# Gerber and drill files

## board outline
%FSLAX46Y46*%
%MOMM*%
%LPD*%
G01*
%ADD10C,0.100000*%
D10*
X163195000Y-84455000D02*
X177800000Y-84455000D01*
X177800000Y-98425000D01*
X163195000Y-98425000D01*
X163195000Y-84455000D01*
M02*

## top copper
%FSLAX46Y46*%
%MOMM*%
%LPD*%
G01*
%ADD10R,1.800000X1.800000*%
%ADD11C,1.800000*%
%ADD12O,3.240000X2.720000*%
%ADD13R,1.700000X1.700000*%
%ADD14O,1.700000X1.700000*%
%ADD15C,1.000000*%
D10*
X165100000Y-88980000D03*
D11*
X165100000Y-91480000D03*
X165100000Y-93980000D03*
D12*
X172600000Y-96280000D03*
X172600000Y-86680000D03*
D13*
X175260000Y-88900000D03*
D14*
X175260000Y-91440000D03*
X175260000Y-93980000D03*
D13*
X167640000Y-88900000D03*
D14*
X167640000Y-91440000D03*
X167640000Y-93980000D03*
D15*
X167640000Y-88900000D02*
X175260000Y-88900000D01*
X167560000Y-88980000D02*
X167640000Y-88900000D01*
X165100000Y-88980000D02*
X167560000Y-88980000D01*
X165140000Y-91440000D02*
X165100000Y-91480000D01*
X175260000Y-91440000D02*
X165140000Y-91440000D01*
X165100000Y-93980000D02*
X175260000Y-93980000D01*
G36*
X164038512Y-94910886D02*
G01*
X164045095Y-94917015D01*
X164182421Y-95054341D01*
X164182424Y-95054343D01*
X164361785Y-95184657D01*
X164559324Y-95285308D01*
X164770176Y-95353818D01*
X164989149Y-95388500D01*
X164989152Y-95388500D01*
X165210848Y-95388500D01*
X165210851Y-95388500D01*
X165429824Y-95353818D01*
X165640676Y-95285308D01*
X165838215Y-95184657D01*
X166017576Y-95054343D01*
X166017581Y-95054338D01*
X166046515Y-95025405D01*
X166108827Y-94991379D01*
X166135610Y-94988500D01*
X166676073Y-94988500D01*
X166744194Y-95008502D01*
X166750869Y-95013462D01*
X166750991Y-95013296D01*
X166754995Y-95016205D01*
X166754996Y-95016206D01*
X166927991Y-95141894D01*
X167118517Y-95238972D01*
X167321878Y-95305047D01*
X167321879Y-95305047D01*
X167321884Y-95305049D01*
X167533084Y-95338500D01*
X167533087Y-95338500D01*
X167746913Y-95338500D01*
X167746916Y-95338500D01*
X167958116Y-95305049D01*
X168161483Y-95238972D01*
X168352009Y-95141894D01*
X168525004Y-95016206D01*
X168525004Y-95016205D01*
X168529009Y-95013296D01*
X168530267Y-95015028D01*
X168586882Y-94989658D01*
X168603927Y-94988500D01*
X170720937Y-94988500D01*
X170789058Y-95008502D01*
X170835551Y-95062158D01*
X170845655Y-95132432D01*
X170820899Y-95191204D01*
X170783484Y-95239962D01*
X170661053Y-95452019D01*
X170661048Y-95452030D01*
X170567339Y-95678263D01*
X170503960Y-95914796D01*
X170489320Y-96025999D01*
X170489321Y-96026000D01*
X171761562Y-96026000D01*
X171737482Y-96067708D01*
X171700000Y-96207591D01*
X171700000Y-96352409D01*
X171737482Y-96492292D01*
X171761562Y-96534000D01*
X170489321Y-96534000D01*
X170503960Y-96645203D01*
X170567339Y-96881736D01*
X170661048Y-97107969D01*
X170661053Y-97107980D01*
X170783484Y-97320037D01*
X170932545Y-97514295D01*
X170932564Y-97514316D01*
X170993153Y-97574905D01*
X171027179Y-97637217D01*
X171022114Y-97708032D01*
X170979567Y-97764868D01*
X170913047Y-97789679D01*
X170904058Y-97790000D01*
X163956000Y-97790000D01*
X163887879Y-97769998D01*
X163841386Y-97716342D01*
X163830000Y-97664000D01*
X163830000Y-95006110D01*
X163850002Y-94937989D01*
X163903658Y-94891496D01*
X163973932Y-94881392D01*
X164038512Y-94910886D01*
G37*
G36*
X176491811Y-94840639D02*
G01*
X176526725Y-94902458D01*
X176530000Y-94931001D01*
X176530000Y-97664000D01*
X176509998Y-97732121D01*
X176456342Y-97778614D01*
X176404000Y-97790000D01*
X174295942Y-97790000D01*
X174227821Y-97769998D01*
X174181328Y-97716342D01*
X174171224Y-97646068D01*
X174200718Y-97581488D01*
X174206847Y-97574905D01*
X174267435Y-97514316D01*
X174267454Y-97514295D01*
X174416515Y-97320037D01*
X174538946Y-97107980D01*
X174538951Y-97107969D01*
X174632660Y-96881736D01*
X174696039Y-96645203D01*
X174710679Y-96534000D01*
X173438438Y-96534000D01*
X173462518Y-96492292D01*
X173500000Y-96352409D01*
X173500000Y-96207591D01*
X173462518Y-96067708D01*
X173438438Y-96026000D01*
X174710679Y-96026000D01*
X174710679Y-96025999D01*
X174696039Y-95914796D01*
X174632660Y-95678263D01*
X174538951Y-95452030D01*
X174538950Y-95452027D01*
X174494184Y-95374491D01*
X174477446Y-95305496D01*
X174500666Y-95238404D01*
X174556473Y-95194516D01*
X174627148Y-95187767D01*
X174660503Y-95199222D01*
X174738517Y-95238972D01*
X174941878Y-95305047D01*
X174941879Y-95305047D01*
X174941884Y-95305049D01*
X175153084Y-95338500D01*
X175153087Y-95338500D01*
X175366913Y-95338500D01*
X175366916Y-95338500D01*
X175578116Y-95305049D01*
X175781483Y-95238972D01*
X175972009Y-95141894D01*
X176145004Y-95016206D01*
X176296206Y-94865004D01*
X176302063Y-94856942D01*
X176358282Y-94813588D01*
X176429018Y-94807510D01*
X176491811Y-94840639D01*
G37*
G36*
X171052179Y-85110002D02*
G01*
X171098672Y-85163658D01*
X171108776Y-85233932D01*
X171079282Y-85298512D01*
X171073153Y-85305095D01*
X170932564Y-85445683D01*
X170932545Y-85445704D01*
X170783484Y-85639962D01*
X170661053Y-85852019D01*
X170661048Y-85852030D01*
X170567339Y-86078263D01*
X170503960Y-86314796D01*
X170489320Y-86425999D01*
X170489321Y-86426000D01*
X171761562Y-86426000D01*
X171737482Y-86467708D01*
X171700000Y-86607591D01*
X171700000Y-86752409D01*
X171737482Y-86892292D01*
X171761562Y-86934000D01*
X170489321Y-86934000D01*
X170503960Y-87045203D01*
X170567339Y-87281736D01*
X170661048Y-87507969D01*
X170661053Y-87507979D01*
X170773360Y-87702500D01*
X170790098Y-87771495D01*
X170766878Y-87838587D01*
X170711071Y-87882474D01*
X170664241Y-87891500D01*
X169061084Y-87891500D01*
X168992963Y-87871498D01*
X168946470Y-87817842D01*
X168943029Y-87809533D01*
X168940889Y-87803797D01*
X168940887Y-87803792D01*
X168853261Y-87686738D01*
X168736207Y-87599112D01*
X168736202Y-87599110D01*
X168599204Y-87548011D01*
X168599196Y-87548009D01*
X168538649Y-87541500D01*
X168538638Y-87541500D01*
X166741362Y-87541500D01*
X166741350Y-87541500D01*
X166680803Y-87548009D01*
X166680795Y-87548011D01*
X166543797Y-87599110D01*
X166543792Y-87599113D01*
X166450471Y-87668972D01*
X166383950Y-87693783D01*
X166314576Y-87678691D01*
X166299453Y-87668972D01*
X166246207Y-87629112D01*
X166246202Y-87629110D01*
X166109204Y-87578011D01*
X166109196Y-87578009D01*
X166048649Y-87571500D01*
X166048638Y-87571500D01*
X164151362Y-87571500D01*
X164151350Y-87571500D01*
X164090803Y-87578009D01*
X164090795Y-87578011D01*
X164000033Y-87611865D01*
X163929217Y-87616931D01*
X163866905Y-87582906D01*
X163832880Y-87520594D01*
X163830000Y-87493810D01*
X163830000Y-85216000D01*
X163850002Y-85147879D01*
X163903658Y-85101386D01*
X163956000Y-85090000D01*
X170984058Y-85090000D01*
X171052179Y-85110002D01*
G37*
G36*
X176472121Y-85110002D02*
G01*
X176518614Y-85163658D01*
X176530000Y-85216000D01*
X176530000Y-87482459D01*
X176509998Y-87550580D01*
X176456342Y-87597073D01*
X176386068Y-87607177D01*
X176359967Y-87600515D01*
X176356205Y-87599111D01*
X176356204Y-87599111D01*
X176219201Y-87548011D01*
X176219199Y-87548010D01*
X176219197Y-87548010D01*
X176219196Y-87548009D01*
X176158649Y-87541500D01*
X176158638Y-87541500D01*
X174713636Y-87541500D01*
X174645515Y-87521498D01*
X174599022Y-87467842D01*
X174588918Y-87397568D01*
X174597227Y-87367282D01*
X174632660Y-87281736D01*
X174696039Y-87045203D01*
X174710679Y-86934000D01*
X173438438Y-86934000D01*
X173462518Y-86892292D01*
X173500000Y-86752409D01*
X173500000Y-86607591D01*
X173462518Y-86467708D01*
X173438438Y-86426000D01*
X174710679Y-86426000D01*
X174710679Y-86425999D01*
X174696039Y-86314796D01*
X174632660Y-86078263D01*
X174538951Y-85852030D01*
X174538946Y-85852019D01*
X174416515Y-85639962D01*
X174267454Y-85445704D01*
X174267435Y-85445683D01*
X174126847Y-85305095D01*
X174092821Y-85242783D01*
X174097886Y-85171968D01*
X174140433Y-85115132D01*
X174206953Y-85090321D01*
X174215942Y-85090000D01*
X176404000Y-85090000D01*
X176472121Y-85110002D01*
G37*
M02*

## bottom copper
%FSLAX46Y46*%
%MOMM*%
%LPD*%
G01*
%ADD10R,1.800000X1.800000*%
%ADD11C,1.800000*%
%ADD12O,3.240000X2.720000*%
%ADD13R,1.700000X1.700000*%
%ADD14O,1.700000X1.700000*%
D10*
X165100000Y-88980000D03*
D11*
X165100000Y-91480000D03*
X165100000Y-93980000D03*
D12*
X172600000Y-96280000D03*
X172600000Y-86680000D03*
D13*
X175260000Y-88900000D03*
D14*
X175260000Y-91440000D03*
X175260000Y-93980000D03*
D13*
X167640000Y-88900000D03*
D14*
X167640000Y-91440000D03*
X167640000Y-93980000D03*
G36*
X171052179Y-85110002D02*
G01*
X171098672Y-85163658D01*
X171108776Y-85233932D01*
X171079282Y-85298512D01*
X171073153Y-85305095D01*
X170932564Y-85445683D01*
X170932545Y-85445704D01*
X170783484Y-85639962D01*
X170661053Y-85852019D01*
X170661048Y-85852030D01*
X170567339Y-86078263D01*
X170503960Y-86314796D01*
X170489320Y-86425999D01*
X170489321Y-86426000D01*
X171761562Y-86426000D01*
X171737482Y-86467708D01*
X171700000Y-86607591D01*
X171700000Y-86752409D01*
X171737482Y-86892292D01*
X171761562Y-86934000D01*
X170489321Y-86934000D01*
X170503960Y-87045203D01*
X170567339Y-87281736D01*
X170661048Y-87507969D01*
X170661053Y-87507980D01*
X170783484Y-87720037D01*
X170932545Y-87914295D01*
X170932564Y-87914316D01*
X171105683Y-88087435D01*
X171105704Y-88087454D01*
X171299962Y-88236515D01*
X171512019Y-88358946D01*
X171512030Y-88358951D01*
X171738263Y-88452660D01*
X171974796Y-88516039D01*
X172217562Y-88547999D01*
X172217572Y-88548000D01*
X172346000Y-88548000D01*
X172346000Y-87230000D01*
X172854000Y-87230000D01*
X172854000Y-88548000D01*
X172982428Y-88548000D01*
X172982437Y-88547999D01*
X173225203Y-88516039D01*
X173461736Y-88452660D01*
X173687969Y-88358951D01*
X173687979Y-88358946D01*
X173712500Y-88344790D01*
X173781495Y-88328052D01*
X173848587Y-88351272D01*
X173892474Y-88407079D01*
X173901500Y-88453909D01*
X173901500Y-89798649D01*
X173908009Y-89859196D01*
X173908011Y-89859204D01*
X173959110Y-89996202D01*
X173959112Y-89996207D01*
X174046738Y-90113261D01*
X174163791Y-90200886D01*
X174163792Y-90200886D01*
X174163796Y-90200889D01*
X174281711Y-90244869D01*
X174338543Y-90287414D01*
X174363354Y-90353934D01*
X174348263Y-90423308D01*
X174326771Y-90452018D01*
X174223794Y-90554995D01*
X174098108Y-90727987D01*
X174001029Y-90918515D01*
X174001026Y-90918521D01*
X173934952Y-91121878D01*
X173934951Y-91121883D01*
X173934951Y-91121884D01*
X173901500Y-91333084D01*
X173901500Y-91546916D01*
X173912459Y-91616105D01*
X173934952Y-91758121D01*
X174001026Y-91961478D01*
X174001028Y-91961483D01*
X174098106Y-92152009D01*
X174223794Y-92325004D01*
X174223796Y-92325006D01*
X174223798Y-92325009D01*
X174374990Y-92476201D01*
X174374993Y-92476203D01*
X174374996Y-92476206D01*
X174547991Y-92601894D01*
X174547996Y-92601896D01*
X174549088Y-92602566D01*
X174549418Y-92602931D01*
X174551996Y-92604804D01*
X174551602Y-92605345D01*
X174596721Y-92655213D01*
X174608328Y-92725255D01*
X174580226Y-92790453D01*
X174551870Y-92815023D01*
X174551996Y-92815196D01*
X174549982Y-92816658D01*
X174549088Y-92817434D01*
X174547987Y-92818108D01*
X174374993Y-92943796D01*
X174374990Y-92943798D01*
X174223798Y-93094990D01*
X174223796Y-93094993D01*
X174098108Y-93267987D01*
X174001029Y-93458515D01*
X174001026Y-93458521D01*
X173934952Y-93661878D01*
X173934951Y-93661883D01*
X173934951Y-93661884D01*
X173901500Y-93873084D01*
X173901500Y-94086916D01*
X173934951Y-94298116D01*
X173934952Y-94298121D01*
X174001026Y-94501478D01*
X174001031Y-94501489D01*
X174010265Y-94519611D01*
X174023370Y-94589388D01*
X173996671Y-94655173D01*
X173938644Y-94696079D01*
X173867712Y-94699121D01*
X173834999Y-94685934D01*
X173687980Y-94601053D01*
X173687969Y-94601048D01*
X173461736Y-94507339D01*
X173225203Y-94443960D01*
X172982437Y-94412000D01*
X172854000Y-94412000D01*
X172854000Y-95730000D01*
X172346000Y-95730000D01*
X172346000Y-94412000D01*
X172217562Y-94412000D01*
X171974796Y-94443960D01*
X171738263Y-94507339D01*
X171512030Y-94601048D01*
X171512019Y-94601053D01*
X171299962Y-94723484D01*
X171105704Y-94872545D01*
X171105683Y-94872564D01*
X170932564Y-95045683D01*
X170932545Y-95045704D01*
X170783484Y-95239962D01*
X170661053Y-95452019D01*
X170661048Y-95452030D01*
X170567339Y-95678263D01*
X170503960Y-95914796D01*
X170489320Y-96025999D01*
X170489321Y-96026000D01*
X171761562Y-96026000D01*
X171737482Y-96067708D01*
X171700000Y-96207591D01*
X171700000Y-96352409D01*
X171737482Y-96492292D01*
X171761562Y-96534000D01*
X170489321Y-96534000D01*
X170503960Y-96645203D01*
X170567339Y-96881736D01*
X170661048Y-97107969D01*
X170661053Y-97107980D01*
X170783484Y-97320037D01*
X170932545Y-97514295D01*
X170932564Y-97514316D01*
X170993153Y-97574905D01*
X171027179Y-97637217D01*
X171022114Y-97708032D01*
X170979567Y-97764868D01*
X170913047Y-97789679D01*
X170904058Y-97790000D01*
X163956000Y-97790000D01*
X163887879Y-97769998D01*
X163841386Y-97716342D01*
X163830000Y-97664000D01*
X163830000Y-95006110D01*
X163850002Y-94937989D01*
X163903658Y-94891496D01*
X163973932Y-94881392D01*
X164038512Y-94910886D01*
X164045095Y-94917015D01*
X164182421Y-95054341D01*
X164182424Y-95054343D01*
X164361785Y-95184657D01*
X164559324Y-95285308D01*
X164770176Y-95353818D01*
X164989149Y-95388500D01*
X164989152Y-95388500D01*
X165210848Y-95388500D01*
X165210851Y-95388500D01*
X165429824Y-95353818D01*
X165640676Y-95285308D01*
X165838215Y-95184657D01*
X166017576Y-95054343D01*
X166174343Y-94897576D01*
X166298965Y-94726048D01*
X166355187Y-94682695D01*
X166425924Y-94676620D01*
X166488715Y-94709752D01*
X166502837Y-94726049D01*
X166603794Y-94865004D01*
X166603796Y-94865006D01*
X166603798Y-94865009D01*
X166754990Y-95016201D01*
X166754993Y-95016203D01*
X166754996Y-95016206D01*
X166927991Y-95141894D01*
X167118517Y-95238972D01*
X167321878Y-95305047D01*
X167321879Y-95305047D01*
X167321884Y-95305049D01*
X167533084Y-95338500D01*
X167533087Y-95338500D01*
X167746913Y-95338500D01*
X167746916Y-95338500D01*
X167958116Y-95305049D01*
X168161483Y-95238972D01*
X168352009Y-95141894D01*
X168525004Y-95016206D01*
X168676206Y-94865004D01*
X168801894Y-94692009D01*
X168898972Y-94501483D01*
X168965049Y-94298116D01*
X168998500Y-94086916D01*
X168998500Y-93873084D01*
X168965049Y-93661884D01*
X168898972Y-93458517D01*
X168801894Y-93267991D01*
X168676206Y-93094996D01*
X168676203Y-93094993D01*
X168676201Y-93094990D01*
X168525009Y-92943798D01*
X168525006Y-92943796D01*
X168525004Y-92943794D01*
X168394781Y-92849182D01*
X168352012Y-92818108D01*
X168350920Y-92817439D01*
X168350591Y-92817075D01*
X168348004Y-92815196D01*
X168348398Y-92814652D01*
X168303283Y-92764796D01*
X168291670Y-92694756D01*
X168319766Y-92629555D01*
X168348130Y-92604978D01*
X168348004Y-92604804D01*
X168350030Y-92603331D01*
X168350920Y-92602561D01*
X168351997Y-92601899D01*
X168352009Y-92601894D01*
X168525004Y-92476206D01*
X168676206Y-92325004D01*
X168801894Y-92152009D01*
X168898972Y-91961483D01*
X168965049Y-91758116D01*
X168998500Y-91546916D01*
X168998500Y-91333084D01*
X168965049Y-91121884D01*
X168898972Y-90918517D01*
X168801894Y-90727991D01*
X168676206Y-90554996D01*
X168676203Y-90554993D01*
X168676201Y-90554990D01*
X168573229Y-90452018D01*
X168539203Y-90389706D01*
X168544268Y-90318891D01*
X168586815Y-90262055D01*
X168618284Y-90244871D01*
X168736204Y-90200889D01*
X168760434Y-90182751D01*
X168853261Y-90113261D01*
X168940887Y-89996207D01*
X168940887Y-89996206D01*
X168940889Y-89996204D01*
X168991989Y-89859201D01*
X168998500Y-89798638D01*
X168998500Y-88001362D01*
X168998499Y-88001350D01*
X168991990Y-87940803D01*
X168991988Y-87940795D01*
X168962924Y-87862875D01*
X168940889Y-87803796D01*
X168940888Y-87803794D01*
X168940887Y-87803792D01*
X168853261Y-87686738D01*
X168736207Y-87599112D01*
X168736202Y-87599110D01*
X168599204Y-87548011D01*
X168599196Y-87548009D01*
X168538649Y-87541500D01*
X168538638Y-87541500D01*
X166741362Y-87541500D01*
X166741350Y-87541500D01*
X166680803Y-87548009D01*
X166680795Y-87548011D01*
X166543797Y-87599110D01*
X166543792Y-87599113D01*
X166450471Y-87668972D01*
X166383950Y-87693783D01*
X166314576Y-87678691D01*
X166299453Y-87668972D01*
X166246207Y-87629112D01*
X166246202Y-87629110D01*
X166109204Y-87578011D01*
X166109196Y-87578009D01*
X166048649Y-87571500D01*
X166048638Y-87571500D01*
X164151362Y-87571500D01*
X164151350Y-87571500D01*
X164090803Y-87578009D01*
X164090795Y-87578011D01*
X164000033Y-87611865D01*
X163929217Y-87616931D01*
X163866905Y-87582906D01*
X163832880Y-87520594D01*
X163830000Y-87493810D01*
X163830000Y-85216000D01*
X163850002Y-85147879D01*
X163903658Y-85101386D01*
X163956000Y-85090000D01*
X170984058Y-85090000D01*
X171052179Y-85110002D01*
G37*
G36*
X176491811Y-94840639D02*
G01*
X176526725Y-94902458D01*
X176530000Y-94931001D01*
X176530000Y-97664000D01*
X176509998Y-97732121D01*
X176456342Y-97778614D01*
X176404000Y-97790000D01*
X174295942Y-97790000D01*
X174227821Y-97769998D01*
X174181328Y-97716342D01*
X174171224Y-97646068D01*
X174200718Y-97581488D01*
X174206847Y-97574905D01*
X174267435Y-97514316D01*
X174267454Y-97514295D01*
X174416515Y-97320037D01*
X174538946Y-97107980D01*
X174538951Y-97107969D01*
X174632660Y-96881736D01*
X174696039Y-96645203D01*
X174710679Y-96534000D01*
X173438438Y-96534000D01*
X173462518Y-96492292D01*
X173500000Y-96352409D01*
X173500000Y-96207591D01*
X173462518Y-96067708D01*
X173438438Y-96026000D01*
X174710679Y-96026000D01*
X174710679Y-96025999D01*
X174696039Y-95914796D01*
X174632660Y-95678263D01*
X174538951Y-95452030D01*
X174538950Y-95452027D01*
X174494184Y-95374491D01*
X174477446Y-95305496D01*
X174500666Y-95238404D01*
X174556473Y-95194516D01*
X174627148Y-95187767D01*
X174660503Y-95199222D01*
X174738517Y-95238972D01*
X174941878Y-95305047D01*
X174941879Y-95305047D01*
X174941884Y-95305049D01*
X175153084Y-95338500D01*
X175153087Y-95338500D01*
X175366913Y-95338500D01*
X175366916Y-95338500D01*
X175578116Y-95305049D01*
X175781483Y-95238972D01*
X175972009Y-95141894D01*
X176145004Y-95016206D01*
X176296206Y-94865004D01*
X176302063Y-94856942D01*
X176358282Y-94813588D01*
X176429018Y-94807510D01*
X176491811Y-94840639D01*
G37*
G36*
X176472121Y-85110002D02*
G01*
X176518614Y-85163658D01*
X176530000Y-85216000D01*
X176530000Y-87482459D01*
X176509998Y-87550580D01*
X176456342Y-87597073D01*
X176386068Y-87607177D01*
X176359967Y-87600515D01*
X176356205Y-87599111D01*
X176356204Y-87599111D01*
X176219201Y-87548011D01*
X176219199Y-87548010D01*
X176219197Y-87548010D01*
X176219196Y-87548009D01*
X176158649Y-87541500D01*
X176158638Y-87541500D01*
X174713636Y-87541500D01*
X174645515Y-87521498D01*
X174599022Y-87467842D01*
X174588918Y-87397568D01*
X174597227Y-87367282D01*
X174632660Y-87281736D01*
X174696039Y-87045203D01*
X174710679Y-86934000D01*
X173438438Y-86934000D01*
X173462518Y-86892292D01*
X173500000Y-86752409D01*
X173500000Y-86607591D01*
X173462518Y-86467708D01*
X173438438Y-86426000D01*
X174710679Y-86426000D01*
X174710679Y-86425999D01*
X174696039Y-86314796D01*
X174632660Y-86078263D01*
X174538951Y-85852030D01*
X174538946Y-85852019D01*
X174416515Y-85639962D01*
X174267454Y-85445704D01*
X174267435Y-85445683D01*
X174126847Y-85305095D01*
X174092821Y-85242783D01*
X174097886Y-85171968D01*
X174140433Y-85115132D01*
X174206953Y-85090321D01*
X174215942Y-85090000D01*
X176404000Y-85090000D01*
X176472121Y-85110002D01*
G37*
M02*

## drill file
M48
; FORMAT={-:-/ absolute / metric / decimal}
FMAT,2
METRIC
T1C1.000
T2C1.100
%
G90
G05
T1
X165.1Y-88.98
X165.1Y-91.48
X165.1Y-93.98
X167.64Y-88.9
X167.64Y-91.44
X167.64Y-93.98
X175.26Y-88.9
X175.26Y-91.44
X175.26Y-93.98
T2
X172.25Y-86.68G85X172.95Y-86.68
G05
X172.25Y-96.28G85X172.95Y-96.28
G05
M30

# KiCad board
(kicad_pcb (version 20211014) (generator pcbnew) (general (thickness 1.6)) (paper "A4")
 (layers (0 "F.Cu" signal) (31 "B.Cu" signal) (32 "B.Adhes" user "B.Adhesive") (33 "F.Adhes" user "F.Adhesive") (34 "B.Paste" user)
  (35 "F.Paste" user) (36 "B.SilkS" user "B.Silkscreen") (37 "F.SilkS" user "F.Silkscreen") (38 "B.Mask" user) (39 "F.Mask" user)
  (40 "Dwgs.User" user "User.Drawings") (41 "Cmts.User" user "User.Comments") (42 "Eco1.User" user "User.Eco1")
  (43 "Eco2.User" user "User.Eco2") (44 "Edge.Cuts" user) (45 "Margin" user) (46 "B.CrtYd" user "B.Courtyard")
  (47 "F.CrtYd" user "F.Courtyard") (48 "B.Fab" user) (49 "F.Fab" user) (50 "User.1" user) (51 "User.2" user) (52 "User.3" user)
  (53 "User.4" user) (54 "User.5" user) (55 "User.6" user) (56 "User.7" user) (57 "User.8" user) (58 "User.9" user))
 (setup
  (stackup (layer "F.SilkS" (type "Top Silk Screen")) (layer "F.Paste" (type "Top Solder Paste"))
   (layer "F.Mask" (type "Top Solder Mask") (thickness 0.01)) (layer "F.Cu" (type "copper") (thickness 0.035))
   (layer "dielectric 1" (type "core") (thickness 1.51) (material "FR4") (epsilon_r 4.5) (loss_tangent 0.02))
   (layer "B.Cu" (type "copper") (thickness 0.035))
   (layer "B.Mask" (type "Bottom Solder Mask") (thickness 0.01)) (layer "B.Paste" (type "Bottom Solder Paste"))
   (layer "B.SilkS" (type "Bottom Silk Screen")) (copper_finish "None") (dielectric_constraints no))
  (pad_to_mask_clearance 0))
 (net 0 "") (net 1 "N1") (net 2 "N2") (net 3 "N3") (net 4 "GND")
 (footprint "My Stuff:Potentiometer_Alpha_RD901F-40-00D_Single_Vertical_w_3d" (layer "F.Cu") (at 165.1 88.98)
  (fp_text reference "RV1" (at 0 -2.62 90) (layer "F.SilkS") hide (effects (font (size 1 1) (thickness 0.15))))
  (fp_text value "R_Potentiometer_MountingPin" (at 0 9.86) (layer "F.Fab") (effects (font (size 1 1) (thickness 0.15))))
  (pad "1" thru_hole rect (at 0 0 90) (size 1.8 1.8) (drill 1) (layers *.Cu *.Mask) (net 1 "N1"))
  (pad "2" thru_hole circle (at 0 2.5 90) (size 1.8 1.8) (drill 1) (layers *.Cu *.Mask) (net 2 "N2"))
  (pad "3" thru_hole circle (at 0 5 90) (size 1.8 1.8) (drill 1) (layers *.Cu *.Mask) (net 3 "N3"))
  (pad "MP" thru_hole oval (at 7.5 7.3 90) (size 2.72 3.24) (drill oval 1.1 1.8) (layers *.Cu *.Mask) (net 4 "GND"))
  (pad "MP" thru_hole oval (at 7.5 -2.3 90) (size 2.72 3.24) (drill oval 1.1 1.8) (layers *.Cu *.Mask) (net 4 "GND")))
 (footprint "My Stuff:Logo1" (layer "F.Cu") (at 171.621669 91.52372 90)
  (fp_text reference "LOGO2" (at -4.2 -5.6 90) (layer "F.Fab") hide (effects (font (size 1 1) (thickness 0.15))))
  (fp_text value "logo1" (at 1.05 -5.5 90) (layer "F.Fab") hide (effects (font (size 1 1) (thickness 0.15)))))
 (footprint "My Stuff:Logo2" (layer "F.Cu") (at 171.64167 91.46628 90)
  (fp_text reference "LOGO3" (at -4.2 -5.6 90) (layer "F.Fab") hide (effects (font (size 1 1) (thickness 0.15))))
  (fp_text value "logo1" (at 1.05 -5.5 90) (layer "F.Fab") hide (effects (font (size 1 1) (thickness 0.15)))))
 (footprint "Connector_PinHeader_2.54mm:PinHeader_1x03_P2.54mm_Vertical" (layer "B.Cu") (at 175.26 88.9 180)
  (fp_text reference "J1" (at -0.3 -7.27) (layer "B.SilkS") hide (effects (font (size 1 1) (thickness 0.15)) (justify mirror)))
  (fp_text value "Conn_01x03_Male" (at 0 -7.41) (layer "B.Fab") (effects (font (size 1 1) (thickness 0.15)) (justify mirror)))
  (pad "1" thru_hole rect locked (at 0 0 180) (size 1.7 1.7) (drill 1) (layers *.Cu *.Mask) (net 1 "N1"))
  (pad "2" thru_hole oval locked (at 0 -2.54 180) (size 1.7 1.7) (drill 1) (layers *.Cu *.Mask) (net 2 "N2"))
  (pad "3" thru_hole oval locked (at 0 -5.08 180) (size 1.7 1.7) (drill 1) (layers *.Cu *.Mask) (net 3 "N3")))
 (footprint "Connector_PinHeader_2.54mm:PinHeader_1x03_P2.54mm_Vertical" (layer "B.Cu") (at 167.64 88.9 180)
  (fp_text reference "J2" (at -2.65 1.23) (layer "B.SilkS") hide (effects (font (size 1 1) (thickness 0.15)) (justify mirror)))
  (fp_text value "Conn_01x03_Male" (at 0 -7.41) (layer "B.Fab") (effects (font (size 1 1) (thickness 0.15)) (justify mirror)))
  (pad "1" thru_hole rect locked (at 0 0 180) (size 1.7 1.7) (drill 1) (layers *.Cu *.Mask) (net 1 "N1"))
  (pad "2" thru_hole oval locked (at 0 -2.54 180) (size 1.7 1.7) (drill 1) (layers *.Cu *.Mask) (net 2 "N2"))
  (pad "3" thru_hole oval locked (at 0 -5.08 180) (size 1.7 1.7) (drill 1) (layers *.Cu *.Mask) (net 3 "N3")))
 (gr_rect (start 163.195 84.455) (end 177.8 98.425) (layer "Edge.Cuts") (width 0.1) (fill none))
 (segment (start 167.64 88.9) (end 175.26 88.9) (width 1) (layer "F.Cu") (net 1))
 (segment (start 167.56 88.98) (end 167.64 88.9) (width 1) (layer "F.Cu") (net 1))
 (segment (start 165.1 88.98) (end 167.56 88.98) (width 1) (layer "F.Cu") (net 1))
 (segment (start 165.14 91.44) (end 165.1 91.48) (width 1) (layer "F.Cu") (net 2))
 (segment (start 175.26 91.44) (end 165.14 91.44) (width 1) (layer "F.Cu") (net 2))
 (segment (start 165.1 93.98) (end 175.26 93.98) (width 1) (layer "F.Cu") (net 3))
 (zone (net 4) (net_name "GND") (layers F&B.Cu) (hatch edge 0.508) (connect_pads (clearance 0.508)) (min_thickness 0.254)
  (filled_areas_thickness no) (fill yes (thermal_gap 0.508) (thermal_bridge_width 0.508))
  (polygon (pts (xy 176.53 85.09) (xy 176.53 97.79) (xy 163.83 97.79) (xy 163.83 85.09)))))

